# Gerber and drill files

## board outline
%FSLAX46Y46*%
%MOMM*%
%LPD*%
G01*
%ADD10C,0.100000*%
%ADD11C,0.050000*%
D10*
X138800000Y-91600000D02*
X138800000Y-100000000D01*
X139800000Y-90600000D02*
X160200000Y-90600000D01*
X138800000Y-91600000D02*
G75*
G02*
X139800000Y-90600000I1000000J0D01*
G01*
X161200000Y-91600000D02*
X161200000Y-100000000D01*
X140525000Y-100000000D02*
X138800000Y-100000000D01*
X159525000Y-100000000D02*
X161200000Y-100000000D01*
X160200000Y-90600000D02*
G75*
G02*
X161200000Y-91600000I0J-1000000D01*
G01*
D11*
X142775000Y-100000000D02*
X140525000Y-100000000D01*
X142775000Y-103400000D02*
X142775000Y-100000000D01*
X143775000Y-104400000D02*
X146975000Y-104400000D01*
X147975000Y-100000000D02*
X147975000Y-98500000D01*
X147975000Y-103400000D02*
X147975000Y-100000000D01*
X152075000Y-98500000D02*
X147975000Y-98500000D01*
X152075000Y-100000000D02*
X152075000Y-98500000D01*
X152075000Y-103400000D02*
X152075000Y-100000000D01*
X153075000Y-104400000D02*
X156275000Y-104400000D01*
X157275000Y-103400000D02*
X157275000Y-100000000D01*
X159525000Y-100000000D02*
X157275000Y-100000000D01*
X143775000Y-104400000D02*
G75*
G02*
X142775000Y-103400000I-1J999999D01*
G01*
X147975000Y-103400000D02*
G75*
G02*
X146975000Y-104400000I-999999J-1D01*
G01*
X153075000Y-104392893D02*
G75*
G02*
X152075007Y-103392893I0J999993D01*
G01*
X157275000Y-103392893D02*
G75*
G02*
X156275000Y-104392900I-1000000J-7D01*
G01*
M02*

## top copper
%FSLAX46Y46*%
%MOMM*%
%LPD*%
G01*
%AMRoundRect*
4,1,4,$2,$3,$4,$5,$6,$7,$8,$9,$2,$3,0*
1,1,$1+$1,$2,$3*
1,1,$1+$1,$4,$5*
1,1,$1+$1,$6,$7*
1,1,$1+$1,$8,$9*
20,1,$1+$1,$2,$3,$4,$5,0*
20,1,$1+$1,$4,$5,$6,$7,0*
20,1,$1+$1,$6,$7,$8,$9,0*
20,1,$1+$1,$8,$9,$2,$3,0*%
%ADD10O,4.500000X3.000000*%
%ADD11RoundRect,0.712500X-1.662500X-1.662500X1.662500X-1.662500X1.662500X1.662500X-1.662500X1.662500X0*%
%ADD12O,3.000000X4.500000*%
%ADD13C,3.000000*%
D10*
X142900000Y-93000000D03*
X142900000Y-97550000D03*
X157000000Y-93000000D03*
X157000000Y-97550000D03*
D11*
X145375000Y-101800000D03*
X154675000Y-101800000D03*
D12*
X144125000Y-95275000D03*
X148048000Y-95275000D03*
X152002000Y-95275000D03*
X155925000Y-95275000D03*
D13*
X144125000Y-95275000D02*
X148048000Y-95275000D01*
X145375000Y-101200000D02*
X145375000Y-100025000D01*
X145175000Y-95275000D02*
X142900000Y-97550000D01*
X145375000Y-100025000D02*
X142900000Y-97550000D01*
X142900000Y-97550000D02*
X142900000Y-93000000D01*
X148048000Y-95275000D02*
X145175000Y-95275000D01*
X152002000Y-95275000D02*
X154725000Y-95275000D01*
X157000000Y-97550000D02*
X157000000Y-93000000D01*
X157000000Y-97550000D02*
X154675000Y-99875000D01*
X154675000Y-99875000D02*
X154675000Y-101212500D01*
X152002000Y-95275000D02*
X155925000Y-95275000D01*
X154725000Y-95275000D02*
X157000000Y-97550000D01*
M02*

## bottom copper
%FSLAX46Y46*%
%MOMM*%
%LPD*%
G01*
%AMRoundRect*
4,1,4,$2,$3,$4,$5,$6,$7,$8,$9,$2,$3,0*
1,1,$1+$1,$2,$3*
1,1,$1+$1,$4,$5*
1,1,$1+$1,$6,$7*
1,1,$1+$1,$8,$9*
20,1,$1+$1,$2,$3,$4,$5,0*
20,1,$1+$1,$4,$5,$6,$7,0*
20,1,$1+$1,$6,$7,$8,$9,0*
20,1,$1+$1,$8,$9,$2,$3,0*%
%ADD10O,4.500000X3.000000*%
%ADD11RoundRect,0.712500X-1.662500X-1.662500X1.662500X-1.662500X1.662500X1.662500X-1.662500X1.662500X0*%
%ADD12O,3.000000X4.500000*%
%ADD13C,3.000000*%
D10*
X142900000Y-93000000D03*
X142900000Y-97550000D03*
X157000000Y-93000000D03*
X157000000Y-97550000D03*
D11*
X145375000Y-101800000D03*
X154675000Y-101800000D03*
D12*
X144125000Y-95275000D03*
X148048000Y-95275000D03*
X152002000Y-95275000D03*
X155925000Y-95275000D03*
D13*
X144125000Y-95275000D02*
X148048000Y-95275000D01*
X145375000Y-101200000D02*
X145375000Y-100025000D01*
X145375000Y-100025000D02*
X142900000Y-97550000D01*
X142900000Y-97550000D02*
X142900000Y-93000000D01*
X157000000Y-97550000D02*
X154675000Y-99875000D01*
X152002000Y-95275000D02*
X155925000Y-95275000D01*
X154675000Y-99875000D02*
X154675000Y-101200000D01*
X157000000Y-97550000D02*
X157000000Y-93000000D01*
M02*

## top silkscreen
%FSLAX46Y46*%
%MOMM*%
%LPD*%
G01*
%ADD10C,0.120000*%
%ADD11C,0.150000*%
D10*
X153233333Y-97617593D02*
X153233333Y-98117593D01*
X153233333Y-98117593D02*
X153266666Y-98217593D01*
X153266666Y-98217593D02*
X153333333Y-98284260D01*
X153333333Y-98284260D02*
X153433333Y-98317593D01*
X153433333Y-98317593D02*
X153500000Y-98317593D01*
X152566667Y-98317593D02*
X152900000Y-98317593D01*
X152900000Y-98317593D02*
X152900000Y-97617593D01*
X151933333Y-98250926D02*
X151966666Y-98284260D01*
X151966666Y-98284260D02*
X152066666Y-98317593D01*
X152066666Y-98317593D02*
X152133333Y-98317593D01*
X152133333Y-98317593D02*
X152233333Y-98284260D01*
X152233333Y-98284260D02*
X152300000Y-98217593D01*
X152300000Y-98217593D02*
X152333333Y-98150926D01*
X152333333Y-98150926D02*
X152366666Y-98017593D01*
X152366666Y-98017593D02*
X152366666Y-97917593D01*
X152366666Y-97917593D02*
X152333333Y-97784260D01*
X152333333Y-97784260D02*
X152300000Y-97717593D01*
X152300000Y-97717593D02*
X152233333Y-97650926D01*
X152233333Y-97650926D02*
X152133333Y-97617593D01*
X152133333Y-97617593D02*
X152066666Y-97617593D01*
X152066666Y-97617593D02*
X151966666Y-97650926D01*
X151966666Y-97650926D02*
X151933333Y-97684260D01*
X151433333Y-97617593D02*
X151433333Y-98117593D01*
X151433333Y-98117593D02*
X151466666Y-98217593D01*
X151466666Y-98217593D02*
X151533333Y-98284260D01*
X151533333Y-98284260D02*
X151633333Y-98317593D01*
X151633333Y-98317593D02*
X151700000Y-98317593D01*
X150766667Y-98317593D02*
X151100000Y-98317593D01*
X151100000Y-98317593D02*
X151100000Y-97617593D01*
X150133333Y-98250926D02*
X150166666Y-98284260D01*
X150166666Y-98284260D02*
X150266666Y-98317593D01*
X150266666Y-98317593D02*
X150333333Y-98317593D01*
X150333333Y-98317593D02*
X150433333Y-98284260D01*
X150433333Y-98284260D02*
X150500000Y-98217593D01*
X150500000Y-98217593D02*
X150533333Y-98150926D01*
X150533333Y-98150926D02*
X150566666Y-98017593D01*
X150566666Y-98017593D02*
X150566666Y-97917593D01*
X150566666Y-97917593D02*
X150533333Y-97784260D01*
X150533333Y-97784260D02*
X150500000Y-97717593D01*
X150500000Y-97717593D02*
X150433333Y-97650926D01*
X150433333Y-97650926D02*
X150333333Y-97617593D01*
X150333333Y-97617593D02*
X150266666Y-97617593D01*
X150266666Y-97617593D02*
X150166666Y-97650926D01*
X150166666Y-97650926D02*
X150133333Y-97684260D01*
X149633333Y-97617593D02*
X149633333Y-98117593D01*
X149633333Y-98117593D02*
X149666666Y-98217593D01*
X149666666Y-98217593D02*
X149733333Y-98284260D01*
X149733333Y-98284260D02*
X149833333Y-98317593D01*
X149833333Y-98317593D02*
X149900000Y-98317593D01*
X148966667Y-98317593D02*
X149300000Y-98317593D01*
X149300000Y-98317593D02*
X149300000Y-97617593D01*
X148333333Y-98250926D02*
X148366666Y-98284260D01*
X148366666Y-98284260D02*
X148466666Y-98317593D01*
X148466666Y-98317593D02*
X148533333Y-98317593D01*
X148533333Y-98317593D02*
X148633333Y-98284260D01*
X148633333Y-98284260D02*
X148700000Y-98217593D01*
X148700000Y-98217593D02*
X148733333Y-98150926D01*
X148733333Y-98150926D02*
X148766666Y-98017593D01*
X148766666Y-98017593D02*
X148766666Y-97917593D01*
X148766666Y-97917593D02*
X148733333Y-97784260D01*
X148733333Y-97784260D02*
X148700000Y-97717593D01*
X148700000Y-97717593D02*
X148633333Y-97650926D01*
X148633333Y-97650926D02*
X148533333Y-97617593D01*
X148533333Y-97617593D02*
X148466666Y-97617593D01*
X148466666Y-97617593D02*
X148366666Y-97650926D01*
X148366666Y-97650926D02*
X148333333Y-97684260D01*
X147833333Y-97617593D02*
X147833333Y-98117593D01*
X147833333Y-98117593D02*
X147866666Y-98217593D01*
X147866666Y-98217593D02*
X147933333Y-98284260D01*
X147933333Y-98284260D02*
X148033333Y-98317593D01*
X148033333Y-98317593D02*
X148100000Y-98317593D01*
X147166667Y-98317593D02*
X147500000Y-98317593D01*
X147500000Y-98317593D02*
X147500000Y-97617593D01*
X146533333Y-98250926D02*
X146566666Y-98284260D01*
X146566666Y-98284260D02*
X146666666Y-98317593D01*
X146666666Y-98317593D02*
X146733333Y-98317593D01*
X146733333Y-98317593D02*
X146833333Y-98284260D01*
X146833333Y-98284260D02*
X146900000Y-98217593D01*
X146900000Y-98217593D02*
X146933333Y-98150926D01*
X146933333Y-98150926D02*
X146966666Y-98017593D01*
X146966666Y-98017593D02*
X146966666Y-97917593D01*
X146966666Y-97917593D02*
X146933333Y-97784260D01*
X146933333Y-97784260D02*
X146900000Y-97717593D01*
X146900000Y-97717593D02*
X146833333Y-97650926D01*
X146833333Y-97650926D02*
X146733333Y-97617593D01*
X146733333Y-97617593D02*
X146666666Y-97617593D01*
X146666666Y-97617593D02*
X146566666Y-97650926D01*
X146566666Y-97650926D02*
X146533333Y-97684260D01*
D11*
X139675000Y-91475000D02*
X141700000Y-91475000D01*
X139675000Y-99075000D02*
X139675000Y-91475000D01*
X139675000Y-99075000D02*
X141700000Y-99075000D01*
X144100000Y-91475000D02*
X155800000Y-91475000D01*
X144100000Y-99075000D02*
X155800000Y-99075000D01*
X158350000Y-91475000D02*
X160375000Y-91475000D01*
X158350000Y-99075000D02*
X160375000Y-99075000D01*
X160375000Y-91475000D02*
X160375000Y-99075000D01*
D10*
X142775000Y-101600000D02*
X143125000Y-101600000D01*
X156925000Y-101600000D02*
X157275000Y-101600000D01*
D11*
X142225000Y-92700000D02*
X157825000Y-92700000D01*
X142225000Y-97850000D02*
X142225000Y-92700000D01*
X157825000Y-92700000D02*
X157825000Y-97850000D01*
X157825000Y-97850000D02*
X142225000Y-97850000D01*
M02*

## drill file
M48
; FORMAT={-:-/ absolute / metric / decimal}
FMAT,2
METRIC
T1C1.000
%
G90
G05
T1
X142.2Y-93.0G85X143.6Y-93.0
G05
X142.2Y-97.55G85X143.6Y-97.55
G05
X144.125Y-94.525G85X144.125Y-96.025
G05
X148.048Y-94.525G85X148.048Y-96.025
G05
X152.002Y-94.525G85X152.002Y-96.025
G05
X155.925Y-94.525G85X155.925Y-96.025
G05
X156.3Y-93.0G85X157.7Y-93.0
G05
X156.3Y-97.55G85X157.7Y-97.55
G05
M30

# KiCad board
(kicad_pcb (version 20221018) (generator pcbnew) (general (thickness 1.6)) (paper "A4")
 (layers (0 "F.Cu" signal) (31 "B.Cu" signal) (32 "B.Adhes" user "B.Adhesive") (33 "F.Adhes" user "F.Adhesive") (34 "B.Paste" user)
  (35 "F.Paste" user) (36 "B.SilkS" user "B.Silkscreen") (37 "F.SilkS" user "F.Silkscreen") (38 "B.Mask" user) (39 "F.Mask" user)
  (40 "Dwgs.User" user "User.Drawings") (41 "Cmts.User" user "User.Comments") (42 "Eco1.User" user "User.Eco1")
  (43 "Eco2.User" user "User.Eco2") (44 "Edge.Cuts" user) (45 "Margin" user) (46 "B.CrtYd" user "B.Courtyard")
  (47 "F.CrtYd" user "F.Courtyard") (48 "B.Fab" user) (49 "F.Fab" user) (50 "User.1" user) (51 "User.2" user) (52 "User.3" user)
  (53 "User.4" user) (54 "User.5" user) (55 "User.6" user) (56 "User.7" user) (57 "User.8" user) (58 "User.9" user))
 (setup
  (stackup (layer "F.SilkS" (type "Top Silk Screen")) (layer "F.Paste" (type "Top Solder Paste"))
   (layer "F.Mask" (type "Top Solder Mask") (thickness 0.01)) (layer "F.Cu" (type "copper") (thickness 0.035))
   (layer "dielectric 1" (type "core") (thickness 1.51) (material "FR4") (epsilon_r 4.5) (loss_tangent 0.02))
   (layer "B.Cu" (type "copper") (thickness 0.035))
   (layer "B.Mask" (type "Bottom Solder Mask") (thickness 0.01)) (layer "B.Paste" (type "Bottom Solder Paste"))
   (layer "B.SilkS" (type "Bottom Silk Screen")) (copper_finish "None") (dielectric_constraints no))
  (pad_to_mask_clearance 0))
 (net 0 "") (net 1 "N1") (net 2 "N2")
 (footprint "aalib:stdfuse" (layer "F.Cu") (at 142.9 93)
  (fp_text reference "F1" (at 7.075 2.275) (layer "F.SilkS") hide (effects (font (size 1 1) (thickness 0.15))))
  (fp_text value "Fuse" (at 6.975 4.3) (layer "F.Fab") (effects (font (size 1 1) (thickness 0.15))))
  (fp_line (start -3.225 -1.525) (end -1.2 -1.525) (stroke (width 0.15) (type solid)) (layer "F.SilkS"))
  (fp_line (start -3.225 6.075) (end -3.225 -1.525) (stroke (width 0.15) (type solid)) (layer "F.SilkS"))
  (fp_line (start -3.225 6.075) (end -1.2 6.075) (stroke (width 0.15) (type solid)) (layer "F.SilkS"))
  (fp_line (start 1.2 -1.525) (end 12.9 -1.525) (stroke (width 0.15) (type solid)) (layer "F.SilkS"))
  (fp_line (start 1.2 6.075) (end 12.9 6.075) (stroke (width 0.15) (type solid)) (layer "F.SilkS"))
  (fp_line (start 15.45 -1.525) (end 17.475 -1.525) (stroke (width 0.15) (type solid)) (layer "F.SilkS"))
  (fp_line (start 15.45 6.075) (end 17.475 6.075) (stroke (width 0.15) (type solid)) (layer "F.SilkS"))
  (fp_line (start 17.475 -1.525) (end 17.475 6.075) (stroke (width 0.15) (type solid)) (layer "F.SilkS"))
  (pad "1" thru_hole oval (at 0 0) (size 4.5 3) (drill oval 2.4 1) (layers "*.Cu" "*.Mask") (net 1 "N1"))
  (pad "1" thru_hole oval (at 0 4.55) (size 4.5 3) (drill oval 2.4 1) (layers "*.Cu" "*.Mask") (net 1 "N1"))
  (pad "2" thru_hole oval (at 14.1 0) (size 4.5 3) (drill oval 2.4 1) (layers "*.Cu" "*.Mask") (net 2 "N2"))
  (pad "2" thru_hole oval (at 14.1 4.55) (size 4.5 3) (drill oval 2.4 1) (layers "*.Cu" "*.Mask") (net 2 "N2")))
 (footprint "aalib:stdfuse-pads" (layer "F.Cu") (at 150.025 100)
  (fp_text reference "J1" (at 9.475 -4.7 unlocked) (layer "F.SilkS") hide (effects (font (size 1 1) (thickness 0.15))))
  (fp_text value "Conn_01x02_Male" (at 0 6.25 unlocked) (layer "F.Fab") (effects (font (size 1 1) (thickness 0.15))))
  (fp_line (start -7.25 1.6) (end -6.9 1.6) (stroke (width 0.12) (type solid)) (layer "F.SilkS"))
  (fp_line (start 6.9 1.6) (end 7.25 1.6) (stroke (width 0.12) (type solid)) (layer "F.SilkS"))
  (fp_line (start -7.25 0) (end -9.5 0) (stroke (width 0.05) (type solid)) (layer "Edge.Cuts"))
  (fp_line (start -7.25 3.4) (end -7.25 0) (stroke (width 0.05) (type solid)) (layer "Edge.Cuts"))
  (fp_line (start -6.25 4.4) (end -3.05 4.4) (stroke (width 0.05) (type solid)) (layer "Edge.Cuts"))
  (fp_line (start -2.05 0) (end -2.05 -1.5) (stroke (width 0.05) (type solid)) (layer "Edge.Cuts"))
  (fp_line (start -2.05 3.4) (end -2.05 0) (stroke (width 0.05) (type solid)) (layer "Edge.Cuts"))
  (fp_line (start 2.05 -1.5) (end -2.05 -1.5) (stroke (width 0.05) (type solid)) (layer "Edge.Cuts"))
  (fp_line (start 2.05 0) (end 2.05 -1.5) (stroke (width 0.05) (type solid)) (layer "Edge.Cuts"))
  (fp_line (start 2.05 3.4) (end 2.05 0) (stroke (width 0.05) (type solid)) (layer "Edge.Cuts"))
  (fp_line (start 3.05 4.4) (end 6.25 4.4) (stroke (width 0.05) (type solid)) (layer "Edge.Cuts"))
  (fp_line (start 7.25 3.4) (end 7.25 0) (stroke (width 0.05) (type solid)) (layer "Edge.Cuts"))
  (fp_line (start 9.5 0) (end 7.25 0) (stroke (width 0.05) (type solid)) (layer "Edge.Cuts"))
  (fp_arc (start -6.25 4.4) (mid -6.957107 4.107107) (end -7.25 3.4) (stroke (width 0.05) (type solid)) (layer "Edge.Cuts"))
  (fp_arc (start -2.05 3.4) (mid -2.342893 4.107107) (end -3.05 4.4) (stroke (width 0.05) (type solid)) (layer "Edge.Cuts"))
  (fp_arc (start 3.05 4.392893) (mid 2.342896 4.099999) (end 2.05 3.392893) (stroke (width 0.05) (type solid)) (layer "Edge.Cuts"))
  (fp_arc (start 7.25 3.392893) (mid 6.957109 4.100004) (end 6.25 4.392893) (stroke (width 0.05) (type solid)) (layer "Edge.Cuts"))
  (pad "1" connect roundrect (at -4.65 1.8) (size 4.75 4.75) (layers "F.Cu" "F.Mask") (roundrect_rratio 0.15) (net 1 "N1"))
  (pad "1" connect roundrect (at -4.65 1.8) (size 4.75 4.75) (layers "B.Cu" "B.Mask") (roundrect_rratio 0.15) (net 1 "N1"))
  (pad "2" connect roundrect (at 4.65 1.8) (size 4.75 4.75) (layers "F.Cu" "F.Mask") (roundrect_rratio 0.15) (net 2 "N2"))
  (pad "2" connect roundrect (at 4.65 1.8) (size 4.75 4.75) (layers "B.Cu" "B.Mask") (roundrect_rratio 0.15) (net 2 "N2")))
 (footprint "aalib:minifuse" (layer "F.Cu") (at 150.025 95.275)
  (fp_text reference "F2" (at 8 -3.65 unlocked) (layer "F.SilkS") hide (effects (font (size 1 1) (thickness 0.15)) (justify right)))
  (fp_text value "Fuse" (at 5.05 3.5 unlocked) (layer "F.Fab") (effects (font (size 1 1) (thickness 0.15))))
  (fp_line (start -7.8 -2.575) (end 7.8 -2.575) (stroke (width 0.15) (type solid)) (layer "F.SilkS"))
  (fp_line (start -7.8 2.575) (end -7.8 -2.575) (stroke (width 0.15) (type solid)) (layer "F.SilkS"))
  (fp_line (start 7.8 -2.575) (end 7.8 2.575) (stroke (width 0.15) (type solid)) (layer "F.SilkS"))
  (fp_line (start 7.8 2.575) (end -7.8 2.575) (stroke (width 0.15) (type solid)) (layer "F.SilkS"))
  (pad "1" thru_hole oval (at -5.9 0) (size 3 4.5) (drill oval 1 2.5) (layers "*.Cu" "*.Mask") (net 1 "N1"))
  (pad "1" thru_hole oval (at -1.977 0) (size 3 4.5) (drill oval 1 2.5) (layers "*.Cu" "*.Mask") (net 1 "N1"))
  (pad "2" thru_hole oval (at 1.977 0) (size 3 4.5) (drill oval 1 2.5) (layers "*.Cu" "*.Mask") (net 2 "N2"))
  (pad "2" thru_hole oval (at 5.9 0) (size 3 4.5) (drill oval 1 2.5) (layers "*.Cu" "*.Mask") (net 2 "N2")))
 (gr_line (start 138.8 91.6) (end 138.8 100) (stroke (width 0.1) (type solid)) (layer "Edge.Cuts"))
 (gr_line (start 139.8 90.6) (end 160.2 90.6) (stroke (width 0.1) (type solid)) (layer "Edge.Cuts"))
 (gr_arc (start 138.8 91.6) (mid 139.092893 90.892893) (end 139.8 90.6) (stroke (width 0.1) (type solid)) (layer "Edge.Cuts"))
 (gr_line (start 161.2 91.6) (end 161.2 100) (stroke (width 0.1) (type solid)) (layer "Edge.Cuts"))
 (gr_line (start 140.525 100) (end 138.8 100) (stroke (width 0.1) (type solid)) (layer "Edge.Cuts"))
 (gr_line (start 159.525 100) (end 161.2 100) (stroke (width 0.1) (type solid)) (layer "Edge.Cuts"))
 (gr_arc (start 160.2 90.6) (mid 160.907107 90.892893) (end 161.2 91.6) (stroke (width 0.1) (type solid)) (layer "Edge.Cuts"))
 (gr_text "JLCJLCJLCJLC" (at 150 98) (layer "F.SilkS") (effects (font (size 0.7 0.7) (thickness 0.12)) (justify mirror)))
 (segment (start 144.125 95.275) (end 148.048 95.275) (width 3) (layer "F.Cu") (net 1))
 (segment (start 145.375 101.2) (end 145.375 100.025) (width 3) (layer "F.Cu") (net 1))
 (segment (start 145.175 95.275) (end 142.9 97.55) (width 3) (layer "F.Cu") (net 1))
 (segment (start 145.375 100.025) (end 142.9 97.55) (width 3) (layer "F.Cu") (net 1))
 (segment (start 142.9 97.55) (end 142.9 93) (width 3) (layer "F.Cu") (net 1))
 (segment (start 148.048 95.275) (end 145.175 95.275) (width 3) (layer "F.Cu") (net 1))
 (segment (start 144.125 95.275) (end 148.048 95.275) (width 3) (layer "B.Cu") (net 1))
 (segment (start 145.375 101.2) (end 145.375 100.025) (width 3) (layer "B.Cu") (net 1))
 (segment (start 145.375 100.025) (end 142.9 97.55) (width 3) (layer "B.Cu") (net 1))
 (segment (start 142.9 97.55) (end 142.9 93) (width 3) (layer "B.Cu") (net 1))
 (segment (start 152.002 95.275) (end 154.725 95.275) (width 3) (layer "F.Cu") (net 2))
 (segment (start 157 97.55) (end 157 93) (width 3) (layer "F.Cu") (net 2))
 (segment (start 157 97.55) (end 154.675 99.875) (width 3) (layer "F.Cu") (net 2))
 (segment (start 154.675 99.875) (end 154.675 101.2125) (width 3) (layer "F.Cu") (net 2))
 (segment (start 152.002 95.275) (end 155.925 95.275) (width 3) (layer "F.Cu") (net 2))
 (segment (start 154.725 95.275) (end 157 97.55) (width 3) (layer "F.Cu") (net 2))
 (segment (start 157 97.55) (end 154.675 99.875) (width 3) (layer "B.Cu") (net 2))
 (segment (start 152.002 95.275) (end 155.925 95.275) (width 3) (layer "B.Cu") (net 2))
 (segment (start 154.675 99.875) (end 154.675 101.2) (width 3) (layer "B.Cu") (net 2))
 (segment (start 157 97.55) (end 157 93) (width 3) (layer "B.Cu") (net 2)))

